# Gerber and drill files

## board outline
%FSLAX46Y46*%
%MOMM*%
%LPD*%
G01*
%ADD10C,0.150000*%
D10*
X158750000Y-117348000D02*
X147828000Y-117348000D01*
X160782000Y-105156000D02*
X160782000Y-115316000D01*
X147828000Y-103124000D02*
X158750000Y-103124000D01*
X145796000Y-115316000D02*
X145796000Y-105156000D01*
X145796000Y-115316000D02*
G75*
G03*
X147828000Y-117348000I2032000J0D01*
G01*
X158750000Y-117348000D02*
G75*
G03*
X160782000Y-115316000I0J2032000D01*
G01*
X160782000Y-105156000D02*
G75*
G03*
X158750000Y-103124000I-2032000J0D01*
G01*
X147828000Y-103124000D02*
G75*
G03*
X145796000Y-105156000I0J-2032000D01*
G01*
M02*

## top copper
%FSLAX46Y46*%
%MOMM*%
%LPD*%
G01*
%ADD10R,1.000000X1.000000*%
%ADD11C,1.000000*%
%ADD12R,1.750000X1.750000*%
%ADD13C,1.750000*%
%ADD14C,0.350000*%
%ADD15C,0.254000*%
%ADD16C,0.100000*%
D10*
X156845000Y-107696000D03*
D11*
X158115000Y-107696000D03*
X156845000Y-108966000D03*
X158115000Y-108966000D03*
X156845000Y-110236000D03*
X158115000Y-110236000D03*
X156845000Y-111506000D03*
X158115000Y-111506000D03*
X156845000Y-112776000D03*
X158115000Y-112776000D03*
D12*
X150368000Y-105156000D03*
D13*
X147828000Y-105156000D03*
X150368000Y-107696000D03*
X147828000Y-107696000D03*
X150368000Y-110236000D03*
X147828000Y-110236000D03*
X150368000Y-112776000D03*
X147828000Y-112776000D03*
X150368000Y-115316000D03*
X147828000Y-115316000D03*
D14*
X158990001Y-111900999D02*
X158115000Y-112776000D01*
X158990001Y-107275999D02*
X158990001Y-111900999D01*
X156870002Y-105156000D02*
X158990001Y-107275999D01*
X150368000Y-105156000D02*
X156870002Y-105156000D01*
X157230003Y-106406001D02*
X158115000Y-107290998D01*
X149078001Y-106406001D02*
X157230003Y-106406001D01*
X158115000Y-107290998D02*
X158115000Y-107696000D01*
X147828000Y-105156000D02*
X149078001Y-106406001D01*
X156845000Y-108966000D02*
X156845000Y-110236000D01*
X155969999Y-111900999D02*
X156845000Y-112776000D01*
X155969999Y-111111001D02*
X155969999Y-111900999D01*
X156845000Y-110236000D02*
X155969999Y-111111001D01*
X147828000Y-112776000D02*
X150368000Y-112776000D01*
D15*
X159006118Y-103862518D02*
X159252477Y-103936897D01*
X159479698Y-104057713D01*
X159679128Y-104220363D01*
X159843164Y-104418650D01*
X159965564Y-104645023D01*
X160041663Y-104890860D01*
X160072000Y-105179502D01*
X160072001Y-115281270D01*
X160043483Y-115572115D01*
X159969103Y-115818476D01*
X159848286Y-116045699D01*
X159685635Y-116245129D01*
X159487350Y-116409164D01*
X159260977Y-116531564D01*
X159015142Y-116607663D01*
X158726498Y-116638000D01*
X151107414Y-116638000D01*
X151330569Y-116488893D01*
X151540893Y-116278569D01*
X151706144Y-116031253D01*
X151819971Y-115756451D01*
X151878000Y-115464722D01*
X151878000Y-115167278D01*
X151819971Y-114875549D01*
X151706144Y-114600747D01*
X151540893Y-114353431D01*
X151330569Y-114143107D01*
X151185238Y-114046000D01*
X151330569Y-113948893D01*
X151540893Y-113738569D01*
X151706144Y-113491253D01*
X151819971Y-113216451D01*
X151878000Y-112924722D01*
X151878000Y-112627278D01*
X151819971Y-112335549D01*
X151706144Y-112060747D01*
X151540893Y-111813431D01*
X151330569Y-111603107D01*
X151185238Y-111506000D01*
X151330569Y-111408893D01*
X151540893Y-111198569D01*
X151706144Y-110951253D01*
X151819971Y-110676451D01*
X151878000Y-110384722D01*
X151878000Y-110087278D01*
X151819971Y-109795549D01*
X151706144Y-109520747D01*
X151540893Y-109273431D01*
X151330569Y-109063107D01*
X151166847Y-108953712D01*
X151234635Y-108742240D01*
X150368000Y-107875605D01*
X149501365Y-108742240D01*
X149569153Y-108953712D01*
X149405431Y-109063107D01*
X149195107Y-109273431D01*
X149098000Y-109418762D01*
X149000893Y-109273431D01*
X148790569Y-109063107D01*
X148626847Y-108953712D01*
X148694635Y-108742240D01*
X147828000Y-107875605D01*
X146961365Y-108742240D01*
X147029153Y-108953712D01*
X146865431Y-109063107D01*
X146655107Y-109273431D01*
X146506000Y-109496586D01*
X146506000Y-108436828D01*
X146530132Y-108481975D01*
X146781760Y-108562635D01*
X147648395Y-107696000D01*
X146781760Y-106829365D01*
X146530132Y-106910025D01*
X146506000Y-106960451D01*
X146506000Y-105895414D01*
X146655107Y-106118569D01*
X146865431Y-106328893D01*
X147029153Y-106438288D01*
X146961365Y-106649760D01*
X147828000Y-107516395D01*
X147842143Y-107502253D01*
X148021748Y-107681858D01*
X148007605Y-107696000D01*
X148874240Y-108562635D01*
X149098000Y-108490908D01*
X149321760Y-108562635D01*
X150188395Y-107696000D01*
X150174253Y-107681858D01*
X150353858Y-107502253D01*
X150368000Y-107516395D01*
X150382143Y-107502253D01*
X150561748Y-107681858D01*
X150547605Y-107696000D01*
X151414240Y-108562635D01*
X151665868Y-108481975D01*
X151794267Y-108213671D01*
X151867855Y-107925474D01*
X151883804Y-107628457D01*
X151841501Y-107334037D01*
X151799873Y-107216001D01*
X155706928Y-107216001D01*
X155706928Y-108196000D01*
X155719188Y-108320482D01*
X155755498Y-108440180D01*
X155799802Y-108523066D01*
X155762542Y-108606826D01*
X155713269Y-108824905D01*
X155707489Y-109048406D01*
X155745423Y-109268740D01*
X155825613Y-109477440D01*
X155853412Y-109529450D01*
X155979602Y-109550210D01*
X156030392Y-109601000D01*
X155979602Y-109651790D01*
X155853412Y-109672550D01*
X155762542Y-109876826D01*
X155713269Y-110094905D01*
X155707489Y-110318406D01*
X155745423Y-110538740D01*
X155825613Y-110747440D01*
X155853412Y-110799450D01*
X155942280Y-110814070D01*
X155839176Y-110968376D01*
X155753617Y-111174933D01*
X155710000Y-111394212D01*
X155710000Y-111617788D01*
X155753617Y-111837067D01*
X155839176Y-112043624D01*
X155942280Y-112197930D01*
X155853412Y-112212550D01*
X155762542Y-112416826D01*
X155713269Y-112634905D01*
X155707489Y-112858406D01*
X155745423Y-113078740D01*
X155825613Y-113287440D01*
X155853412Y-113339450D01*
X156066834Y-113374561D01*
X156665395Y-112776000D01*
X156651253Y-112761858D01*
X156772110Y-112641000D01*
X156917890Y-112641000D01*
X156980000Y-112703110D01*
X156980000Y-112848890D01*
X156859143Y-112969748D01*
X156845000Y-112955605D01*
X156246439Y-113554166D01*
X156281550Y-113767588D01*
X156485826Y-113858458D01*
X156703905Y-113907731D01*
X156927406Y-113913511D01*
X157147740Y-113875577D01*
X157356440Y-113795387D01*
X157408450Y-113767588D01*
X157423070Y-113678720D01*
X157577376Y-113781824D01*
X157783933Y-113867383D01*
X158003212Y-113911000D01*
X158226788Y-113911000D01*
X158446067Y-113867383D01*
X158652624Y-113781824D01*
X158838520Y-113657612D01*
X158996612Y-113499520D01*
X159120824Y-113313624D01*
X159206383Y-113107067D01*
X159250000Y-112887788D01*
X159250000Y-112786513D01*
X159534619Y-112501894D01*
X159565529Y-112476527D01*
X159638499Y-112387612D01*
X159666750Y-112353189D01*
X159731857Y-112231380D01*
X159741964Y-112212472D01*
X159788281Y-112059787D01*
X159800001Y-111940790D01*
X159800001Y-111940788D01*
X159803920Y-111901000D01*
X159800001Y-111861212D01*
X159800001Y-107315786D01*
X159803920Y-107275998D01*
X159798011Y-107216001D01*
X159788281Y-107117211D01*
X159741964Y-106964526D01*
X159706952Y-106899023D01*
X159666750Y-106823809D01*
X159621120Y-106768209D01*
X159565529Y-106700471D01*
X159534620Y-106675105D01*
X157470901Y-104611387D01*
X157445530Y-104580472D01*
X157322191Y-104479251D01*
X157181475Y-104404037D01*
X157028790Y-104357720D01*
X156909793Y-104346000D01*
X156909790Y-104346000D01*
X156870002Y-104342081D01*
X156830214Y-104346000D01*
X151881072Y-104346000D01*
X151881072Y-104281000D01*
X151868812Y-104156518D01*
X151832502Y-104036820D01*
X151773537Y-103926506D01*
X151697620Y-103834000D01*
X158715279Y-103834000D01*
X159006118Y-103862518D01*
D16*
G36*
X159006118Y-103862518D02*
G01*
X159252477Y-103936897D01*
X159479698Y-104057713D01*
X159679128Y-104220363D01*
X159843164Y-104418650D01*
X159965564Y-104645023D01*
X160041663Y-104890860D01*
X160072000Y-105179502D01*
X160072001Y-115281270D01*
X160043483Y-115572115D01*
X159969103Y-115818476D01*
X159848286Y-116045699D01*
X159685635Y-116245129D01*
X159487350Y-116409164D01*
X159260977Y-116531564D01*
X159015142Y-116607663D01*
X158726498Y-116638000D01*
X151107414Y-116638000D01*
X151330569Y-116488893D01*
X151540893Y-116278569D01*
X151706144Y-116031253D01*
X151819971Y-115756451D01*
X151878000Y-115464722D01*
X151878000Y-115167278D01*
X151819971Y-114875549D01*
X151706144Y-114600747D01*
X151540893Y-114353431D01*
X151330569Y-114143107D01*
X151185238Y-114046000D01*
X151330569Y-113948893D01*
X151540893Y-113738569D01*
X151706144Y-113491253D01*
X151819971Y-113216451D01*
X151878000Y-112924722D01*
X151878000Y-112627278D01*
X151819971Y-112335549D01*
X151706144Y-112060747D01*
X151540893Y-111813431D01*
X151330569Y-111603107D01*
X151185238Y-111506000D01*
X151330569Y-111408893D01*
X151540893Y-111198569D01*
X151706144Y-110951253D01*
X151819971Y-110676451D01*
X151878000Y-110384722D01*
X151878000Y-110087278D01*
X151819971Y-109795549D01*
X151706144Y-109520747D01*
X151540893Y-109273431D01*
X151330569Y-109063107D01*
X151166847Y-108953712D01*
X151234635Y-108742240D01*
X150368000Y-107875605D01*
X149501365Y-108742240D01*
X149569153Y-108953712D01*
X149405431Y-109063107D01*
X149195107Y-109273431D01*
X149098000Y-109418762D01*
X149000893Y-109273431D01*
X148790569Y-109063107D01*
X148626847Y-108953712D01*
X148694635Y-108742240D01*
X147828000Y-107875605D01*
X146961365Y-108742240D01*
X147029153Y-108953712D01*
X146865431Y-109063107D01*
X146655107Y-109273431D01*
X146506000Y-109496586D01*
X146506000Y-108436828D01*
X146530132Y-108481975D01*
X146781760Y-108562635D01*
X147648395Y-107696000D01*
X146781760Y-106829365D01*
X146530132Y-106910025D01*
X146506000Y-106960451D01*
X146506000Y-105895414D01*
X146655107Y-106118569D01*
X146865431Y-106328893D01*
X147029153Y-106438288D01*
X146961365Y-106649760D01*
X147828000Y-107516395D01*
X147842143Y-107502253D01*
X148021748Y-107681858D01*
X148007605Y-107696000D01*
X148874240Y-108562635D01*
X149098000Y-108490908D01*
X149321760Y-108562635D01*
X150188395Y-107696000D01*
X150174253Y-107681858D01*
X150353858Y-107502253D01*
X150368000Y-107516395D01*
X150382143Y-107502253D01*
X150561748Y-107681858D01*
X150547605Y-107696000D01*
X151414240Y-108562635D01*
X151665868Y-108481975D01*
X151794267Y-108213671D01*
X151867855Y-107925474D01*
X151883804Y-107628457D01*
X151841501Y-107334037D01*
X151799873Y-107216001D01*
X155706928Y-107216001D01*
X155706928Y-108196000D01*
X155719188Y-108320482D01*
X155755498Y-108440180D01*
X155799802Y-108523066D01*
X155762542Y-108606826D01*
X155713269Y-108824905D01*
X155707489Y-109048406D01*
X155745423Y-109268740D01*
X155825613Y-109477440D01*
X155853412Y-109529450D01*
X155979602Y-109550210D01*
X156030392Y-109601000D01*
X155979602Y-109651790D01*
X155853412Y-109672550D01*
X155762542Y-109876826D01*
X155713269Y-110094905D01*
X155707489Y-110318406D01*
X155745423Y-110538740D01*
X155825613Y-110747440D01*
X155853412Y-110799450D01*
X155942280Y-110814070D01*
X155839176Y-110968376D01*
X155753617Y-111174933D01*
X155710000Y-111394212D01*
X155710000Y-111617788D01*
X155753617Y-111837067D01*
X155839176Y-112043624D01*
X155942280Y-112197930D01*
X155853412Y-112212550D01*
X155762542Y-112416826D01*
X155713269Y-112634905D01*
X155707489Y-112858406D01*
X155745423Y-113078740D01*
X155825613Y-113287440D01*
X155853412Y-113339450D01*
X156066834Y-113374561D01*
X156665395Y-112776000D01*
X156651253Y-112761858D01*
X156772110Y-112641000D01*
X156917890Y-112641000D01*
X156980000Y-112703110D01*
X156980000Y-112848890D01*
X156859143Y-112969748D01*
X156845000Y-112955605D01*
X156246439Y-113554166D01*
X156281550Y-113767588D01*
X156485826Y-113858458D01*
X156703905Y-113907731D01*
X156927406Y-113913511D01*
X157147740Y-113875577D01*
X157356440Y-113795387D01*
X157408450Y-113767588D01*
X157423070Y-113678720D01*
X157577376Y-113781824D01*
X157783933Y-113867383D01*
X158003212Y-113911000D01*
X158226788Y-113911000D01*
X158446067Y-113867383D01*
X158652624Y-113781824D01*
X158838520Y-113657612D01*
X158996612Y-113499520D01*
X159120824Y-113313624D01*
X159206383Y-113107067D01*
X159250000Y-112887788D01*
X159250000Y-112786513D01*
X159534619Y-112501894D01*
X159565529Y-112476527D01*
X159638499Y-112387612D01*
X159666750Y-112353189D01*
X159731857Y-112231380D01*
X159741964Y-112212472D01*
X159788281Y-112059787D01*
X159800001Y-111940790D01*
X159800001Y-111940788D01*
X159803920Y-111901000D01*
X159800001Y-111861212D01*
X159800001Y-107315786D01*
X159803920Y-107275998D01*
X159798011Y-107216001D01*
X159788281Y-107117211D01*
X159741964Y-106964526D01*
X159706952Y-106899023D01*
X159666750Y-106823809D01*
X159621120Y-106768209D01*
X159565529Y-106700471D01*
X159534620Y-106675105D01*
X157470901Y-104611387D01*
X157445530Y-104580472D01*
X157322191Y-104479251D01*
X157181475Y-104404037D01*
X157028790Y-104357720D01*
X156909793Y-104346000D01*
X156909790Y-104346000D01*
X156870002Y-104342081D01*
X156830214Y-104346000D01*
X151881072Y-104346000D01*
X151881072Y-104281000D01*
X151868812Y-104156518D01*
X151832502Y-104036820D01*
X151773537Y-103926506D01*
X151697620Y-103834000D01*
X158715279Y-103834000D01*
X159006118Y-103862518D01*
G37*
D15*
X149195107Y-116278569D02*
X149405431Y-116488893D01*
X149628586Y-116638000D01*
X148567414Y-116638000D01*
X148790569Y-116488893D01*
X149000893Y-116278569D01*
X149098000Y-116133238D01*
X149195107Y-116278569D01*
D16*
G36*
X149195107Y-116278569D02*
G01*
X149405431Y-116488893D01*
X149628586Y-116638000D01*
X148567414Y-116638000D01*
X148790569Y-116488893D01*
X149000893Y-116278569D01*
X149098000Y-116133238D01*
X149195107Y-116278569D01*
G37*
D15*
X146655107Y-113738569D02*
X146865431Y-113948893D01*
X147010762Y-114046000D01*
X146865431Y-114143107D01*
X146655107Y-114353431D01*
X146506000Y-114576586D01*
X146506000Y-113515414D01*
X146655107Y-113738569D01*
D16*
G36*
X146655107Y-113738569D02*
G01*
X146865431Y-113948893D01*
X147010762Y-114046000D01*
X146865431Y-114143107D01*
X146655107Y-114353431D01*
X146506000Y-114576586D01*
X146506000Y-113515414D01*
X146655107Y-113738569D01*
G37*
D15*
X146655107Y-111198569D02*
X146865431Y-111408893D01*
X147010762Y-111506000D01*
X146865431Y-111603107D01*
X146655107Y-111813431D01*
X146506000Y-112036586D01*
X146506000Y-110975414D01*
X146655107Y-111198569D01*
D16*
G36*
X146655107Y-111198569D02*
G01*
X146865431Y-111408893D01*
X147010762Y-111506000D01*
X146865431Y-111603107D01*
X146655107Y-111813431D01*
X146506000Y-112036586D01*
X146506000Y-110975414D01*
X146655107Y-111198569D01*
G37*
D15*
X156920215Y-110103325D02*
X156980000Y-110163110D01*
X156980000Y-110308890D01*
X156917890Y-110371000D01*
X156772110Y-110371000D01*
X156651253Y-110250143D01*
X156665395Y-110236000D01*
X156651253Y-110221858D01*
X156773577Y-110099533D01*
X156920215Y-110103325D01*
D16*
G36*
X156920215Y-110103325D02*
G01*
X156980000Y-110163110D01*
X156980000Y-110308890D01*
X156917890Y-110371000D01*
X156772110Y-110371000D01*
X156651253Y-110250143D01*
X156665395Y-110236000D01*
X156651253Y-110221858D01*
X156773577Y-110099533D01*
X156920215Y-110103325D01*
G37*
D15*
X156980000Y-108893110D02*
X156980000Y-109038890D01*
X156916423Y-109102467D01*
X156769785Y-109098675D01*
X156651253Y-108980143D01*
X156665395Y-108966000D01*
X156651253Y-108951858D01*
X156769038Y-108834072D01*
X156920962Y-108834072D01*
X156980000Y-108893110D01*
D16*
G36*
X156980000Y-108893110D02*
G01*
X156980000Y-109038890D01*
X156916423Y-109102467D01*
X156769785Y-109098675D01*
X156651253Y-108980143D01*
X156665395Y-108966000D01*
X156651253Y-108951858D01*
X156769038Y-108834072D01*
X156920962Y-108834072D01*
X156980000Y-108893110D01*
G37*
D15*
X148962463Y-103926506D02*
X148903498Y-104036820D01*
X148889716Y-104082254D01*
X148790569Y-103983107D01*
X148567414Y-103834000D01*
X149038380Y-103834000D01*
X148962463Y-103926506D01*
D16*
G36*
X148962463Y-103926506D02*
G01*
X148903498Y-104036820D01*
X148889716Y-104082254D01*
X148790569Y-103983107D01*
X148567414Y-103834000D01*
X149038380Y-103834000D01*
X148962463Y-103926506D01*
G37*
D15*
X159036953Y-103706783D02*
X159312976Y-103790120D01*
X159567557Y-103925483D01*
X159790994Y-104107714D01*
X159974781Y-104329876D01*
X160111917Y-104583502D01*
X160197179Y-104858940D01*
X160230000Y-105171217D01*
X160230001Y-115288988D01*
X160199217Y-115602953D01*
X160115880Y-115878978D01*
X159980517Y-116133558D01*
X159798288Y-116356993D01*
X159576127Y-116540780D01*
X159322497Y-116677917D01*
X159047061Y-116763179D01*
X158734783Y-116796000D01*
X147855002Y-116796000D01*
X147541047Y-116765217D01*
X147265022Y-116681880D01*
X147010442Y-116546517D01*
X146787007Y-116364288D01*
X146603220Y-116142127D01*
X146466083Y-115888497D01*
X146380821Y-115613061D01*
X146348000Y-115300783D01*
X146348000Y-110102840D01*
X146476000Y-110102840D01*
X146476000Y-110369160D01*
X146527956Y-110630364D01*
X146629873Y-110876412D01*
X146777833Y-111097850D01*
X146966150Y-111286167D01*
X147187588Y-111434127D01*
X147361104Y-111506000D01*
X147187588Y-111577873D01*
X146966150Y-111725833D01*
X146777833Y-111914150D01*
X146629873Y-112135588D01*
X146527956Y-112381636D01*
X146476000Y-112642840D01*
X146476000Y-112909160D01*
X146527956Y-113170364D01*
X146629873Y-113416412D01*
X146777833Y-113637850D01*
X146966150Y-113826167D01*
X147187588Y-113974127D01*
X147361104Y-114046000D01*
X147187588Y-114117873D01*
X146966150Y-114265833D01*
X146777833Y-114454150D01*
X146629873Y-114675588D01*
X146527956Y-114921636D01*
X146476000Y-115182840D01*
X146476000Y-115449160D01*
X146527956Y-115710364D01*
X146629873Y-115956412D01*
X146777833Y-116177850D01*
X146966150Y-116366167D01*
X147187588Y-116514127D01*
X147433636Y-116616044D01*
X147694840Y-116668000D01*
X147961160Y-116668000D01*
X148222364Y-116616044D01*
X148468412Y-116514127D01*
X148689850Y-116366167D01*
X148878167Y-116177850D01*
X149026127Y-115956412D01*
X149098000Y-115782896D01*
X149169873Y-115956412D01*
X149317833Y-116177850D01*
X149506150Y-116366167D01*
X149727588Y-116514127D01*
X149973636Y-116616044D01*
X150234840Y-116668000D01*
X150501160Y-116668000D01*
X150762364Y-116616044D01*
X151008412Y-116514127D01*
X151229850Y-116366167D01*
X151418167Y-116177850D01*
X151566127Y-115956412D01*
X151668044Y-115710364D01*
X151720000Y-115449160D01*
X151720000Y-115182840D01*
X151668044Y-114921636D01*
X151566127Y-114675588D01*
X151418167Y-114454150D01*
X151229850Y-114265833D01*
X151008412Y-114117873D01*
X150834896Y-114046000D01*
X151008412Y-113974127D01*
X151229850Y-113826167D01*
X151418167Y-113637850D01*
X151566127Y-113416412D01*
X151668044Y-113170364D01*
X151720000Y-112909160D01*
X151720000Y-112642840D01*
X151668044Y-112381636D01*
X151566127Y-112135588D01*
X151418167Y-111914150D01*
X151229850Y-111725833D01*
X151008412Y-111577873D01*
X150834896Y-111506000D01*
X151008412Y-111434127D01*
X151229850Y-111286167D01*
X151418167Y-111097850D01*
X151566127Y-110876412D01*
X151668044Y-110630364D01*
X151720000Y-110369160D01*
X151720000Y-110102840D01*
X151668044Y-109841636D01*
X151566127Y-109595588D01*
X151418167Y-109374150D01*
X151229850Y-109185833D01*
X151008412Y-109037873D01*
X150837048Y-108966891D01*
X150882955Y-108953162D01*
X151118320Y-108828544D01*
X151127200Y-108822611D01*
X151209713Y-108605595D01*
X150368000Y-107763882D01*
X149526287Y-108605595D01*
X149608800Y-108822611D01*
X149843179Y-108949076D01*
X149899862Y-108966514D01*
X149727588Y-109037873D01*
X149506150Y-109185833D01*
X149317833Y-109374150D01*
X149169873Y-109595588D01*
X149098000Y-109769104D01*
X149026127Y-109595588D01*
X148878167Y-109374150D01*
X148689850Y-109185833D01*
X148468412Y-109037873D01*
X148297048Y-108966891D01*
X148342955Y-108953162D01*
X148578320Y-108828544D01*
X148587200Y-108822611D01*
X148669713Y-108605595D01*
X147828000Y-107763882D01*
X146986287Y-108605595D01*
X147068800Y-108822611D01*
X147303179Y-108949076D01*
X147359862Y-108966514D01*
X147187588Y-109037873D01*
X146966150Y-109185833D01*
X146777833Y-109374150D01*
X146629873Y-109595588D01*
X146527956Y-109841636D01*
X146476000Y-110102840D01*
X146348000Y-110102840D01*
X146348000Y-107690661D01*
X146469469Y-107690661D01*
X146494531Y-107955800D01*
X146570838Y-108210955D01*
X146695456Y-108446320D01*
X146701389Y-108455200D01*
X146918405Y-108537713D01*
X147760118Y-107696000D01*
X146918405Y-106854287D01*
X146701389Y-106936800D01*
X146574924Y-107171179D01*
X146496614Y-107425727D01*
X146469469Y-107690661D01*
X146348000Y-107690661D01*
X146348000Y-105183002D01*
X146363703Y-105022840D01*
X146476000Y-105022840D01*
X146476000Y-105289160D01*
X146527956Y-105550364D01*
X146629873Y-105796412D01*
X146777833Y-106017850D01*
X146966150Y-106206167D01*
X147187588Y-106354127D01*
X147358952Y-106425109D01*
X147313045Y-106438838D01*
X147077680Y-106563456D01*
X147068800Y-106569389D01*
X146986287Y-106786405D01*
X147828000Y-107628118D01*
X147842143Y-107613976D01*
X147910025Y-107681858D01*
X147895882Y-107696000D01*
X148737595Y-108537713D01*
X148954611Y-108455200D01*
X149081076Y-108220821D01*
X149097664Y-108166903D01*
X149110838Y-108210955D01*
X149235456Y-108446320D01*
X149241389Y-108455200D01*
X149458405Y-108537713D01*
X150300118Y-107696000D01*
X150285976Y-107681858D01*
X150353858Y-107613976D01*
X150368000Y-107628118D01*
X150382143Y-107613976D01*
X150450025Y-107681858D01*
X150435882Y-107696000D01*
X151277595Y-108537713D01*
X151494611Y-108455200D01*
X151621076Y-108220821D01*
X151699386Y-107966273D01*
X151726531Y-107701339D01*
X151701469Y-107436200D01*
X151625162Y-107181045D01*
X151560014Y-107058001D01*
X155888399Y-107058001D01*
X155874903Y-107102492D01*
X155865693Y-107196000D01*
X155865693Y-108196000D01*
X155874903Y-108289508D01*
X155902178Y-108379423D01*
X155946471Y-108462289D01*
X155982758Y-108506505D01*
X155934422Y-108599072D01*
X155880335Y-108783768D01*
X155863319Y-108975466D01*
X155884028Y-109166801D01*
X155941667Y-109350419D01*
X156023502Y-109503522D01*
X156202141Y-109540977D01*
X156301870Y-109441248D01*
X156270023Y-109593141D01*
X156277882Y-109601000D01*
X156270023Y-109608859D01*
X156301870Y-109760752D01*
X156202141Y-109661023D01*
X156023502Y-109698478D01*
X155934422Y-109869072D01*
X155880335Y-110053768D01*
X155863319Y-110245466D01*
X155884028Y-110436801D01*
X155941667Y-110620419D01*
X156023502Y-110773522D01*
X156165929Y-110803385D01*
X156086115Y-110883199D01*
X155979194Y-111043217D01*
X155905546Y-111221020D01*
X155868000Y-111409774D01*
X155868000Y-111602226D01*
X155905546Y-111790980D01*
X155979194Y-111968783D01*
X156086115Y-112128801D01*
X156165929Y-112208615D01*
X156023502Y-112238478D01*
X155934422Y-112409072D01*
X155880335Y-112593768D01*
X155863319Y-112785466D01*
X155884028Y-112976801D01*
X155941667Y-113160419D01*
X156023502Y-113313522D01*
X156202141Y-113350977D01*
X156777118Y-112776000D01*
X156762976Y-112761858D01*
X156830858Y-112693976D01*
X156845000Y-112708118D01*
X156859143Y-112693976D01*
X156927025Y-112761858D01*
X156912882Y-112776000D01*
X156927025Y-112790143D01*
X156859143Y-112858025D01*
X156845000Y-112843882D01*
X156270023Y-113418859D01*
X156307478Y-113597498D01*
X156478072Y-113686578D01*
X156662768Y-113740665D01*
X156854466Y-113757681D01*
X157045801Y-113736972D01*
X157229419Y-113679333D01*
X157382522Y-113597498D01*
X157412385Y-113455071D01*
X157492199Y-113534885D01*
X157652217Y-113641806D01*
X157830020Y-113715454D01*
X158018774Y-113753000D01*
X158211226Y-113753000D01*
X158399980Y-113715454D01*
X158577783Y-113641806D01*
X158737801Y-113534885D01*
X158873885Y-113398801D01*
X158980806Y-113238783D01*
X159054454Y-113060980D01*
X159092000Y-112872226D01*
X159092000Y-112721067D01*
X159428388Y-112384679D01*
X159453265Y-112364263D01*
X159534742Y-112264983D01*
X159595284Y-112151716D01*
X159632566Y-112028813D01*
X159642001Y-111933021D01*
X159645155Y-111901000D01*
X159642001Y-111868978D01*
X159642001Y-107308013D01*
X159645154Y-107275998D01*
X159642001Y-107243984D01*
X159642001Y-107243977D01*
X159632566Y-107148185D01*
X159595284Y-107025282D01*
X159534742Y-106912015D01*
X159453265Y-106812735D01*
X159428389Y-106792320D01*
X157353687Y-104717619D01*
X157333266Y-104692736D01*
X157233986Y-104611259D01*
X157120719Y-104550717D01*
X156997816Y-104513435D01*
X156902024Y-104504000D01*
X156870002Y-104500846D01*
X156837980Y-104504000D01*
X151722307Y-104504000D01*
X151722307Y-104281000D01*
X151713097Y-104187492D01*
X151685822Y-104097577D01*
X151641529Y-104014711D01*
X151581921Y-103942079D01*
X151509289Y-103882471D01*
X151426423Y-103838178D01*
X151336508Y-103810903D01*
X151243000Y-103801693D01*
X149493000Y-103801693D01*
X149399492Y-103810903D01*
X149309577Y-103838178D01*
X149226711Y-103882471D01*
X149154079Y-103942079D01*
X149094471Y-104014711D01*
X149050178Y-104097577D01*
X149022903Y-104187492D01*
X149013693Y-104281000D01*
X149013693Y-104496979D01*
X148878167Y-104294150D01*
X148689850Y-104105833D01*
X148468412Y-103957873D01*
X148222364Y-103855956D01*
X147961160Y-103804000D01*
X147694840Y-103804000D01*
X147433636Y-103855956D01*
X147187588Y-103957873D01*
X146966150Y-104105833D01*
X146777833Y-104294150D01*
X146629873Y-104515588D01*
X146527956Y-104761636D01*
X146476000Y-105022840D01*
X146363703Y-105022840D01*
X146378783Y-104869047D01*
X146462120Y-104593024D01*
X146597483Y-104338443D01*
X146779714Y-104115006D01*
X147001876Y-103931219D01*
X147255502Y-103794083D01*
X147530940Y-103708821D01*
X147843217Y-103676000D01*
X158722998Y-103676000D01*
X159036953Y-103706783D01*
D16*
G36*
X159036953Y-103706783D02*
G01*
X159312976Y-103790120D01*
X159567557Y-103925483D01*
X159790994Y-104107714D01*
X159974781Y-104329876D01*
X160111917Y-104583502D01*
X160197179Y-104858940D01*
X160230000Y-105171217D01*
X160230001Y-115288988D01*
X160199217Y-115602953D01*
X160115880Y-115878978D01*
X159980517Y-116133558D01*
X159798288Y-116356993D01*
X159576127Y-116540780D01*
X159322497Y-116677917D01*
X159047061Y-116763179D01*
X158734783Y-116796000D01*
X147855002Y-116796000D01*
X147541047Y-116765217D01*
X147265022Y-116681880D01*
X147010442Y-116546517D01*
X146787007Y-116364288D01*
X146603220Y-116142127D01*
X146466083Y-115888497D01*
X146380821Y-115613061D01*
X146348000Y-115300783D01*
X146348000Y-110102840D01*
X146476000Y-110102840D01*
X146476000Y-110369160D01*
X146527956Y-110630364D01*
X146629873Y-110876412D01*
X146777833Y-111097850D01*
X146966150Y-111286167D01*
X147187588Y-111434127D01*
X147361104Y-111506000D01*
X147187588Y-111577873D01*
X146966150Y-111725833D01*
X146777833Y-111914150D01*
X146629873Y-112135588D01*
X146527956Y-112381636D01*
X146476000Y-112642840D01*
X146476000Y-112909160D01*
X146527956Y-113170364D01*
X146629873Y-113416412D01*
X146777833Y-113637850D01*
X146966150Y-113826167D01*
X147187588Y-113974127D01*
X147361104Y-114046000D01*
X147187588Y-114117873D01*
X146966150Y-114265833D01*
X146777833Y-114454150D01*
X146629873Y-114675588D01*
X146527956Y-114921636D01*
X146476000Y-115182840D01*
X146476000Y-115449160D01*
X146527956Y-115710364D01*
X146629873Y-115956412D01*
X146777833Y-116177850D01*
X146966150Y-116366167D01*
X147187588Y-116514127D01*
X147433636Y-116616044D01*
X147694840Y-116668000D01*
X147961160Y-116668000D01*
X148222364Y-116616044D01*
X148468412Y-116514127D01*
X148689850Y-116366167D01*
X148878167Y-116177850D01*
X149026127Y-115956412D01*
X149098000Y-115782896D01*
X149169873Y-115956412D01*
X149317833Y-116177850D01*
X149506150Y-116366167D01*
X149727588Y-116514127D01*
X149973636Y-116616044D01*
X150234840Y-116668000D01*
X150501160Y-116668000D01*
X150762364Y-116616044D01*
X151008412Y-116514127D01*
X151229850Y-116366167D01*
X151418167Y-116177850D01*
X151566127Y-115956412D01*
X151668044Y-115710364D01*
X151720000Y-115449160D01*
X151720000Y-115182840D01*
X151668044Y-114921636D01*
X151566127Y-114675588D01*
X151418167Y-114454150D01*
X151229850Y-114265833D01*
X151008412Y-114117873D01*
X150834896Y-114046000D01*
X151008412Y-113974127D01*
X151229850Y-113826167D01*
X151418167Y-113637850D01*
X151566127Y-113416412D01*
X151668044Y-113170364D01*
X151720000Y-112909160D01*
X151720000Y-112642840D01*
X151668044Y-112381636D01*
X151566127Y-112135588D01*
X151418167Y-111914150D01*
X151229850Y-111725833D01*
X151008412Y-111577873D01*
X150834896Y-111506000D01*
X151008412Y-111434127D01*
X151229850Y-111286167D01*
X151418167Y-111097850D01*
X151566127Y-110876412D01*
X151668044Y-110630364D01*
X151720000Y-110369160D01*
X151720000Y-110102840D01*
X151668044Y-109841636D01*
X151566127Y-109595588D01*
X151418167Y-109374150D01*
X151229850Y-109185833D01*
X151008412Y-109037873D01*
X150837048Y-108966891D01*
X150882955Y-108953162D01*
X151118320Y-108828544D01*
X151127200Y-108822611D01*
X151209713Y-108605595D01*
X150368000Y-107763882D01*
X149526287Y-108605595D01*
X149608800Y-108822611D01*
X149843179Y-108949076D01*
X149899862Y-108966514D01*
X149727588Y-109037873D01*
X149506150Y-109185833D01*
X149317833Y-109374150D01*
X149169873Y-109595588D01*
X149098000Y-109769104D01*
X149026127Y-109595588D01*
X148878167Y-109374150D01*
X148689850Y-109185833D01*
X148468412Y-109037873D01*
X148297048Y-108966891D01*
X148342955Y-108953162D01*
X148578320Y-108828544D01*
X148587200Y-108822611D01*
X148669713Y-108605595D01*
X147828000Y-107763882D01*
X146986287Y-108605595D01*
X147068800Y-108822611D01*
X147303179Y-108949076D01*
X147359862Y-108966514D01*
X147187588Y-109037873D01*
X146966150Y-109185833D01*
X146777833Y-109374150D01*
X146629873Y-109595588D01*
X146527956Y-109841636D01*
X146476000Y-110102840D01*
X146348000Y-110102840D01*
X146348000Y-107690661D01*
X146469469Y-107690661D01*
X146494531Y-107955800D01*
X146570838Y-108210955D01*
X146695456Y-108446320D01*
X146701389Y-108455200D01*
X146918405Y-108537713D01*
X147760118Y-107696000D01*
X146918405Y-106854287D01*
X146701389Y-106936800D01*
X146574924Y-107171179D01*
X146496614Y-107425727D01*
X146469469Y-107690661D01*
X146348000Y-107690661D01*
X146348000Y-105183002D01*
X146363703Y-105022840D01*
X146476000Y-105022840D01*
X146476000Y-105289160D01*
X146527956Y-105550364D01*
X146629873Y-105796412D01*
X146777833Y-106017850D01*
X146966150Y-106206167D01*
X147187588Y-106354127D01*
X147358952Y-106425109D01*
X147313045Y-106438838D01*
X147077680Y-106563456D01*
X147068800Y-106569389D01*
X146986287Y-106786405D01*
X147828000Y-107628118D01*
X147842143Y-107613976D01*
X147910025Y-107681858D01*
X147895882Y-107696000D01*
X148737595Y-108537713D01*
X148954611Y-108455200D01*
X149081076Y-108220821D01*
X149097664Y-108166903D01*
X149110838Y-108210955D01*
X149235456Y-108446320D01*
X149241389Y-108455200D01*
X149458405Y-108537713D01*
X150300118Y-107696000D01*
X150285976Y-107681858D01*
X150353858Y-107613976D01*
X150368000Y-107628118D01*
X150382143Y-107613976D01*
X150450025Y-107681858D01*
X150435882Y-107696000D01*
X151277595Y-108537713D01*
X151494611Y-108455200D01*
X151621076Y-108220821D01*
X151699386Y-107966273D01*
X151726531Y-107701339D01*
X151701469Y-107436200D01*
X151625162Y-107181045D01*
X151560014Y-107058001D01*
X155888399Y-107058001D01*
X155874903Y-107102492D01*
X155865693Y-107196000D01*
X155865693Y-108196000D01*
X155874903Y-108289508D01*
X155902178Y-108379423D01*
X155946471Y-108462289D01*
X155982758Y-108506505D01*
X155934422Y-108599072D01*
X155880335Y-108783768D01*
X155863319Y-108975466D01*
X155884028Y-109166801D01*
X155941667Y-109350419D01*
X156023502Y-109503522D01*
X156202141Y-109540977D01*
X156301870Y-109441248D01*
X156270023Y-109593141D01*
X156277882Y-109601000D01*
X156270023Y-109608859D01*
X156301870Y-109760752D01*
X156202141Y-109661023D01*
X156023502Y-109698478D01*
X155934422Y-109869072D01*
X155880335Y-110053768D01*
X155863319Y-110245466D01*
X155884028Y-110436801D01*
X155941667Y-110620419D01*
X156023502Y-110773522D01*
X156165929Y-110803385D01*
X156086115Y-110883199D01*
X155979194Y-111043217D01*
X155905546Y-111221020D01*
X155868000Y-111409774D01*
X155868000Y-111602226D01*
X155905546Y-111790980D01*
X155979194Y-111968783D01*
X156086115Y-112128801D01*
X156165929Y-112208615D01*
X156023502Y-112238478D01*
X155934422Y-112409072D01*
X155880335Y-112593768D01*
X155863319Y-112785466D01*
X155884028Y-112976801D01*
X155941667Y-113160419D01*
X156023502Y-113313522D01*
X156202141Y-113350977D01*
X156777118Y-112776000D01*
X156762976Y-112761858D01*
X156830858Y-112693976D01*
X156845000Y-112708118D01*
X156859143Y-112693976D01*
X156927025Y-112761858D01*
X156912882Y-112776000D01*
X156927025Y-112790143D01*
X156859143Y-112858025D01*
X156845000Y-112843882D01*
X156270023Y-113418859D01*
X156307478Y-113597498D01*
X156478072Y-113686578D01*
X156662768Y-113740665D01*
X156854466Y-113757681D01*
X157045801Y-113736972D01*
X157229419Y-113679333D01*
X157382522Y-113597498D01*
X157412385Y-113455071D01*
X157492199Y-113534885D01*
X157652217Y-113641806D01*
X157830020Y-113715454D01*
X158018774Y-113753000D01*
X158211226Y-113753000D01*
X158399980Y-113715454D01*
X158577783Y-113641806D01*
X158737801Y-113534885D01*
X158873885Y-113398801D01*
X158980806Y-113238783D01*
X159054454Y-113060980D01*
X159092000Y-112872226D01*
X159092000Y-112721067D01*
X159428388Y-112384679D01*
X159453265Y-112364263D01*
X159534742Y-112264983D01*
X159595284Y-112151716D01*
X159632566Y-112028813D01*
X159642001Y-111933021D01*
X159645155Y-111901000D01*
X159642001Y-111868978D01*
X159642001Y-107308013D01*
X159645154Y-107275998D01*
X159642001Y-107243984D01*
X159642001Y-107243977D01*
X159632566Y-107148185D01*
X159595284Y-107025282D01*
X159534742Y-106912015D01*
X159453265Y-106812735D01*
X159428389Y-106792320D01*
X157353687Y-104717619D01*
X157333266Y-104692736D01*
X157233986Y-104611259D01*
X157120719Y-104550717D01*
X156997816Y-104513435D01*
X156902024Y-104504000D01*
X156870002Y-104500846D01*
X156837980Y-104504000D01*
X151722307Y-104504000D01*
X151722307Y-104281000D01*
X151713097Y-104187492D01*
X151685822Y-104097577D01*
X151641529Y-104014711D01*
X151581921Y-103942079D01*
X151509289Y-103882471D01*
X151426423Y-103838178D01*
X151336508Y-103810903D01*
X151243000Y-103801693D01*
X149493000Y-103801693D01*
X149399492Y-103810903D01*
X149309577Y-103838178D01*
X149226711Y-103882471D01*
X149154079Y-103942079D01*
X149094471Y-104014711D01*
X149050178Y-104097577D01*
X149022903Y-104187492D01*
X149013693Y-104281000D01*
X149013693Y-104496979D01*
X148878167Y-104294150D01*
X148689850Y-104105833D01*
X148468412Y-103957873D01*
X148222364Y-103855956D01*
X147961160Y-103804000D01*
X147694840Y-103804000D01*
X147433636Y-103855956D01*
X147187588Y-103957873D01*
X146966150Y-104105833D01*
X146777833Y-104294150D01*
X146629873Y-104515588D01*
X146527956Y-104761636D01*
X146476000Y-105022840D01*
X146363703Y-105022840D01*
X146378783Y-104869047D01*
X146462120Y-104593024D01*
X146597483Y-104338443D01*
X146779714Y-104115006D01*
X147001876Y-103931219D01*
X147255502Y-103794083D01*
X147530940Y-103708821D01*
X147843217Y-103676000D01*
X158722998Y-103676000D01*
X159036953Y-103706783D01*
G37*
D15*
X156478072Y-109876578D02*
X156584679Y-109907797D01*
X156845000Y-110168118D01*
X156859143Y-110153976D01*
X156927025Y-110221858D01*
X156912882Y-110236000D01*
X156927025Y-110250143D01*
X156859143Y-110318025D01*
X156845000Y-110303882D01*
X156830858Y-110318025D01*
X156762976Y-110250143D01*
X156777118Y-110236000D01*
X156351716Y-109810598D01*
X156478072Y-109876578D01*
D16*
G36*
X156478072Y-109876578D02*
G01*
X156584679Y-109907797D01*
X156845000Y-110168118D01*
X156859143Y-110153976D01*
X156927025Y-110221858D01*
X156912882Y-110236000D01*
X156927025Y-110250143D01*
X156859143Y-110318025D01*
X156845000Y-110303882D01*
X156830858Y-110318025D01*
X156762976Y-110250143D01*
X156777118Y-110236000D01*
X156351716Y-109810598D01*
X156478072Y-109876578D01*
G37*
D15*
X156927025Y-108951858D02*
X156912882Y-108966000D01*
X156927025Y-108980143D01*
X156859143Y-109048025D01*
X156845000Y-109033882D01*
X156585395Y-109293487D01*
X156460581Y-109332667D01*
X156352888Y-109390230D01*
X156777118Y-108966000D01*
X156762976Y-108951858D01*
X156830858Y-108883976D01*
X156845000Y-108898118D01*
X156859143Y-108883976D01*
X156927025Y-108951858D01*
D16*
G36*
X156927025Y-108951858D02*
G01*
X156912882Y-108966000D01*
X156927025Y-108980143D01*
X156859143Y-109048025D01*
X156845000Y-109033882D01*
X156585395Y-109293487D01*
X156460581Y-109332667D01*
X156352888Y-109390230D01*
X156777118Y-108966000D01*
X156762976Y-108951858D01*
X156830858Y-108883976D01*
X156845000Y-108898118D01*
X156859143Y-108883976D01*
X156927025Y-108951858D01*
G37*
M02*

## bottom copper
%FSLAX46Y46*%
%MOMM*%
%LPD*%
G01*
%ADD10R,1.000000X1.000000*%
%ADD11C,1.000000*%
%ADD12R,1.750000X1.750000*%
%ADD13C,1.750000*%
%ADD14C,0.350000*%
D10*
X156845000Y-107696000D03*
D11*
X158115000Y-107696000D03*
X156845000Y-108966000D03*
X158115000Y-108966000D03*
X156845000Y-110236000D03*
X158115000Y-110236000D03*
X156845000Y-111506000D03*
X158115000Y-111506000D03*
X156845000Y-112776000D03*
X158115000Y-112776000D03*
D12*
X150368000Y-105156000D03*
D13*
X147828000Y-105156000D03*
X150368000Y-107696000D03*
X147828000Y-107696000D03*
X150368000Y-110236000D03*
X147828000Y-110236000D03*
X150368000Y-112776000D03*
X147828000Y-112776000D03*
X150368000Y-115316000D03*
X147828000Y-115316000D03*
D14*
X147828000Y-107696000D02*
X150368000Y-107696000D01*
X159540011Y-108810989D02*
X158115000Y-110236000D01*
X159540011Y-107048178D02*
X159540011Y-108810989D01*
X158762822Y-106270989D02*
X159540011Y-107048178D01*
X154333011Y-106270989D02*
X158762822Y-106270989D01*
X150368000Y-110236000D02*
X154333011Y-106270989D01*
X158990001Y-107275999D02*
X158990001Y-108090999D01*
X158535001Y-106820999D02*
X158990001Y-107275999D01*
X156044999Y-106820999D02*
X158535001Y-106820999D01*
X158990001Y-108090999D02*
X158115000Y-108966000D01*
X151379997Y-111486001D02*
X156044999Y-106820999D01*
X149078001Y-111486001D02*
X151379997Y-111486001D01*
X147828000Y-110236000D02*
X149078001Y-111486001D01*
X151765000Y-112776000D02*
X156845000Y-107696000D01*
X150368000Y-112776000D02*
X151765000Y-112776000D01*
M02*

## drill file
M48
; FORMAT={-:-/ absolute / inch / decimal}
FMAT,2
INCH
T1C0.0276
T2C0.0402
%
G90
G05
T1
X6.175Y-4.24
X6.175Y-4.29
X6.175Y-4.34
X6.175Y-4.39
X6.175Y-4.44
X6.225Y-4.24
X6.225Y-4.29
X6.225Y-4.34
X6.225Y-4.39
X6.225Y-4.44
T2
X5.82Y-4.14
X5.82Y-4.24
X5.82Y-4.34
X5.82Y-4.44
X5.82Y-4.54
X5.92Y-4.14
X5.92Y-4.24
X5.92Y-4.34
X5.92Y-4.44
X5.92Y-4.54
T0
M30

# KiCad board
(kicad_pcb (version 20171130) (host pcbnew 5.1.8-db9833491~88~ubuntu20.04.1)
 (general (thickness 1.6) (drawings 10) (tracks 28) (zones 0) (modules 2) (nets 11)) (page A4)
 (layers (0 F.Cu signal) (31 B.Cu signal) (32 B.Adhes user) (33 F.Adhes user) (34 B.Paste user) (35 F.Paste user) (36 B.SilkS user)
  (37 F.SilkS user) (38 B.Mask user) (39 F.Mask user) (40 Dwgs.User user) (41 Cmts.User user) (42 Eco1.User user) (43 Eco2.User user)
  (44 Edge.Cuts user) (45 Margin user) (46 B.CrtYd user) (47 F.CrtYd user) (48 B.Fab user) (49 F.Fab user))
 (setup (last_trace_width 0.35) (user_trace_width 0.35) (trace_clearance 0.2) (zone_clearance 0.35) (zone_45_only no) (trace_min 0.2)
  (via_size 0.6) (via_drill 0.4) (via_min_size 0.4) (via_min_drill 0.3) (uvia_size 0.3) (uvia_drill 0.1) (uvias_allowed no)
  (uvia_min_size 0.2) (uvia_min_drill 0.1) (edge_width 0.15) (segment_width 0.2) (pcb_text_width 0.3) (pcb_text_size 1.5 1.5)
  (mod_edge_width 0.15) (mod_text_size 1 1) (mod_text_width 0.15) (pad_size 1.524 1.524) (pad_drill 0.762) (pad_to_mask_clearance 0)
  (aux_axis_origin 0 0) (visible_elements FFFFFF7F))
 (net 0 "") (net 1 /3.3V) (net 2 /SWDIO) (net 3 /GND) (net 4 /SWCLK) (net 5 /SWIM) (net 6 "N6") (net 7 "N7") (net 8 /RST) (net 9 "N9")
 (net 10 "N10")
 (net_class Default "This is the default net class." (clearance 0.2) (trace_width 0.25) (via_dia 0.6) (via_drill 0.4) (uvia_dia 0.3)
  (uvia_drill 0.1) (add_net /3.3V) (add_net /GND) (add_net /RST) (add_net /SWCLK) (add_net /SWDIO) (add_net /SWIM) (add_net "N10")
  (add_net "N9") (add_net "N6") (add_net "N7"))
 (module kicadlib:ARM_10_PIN (layer F.Cu) (at 157.48 110.236)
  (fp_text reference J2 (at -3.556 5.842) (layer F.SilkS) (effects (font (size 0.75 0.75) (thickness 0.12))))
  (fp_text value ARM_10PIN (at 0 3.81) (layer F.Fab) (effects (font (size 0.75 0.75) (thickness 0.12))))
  (pad 1 thru_hole rect (at -0.635 -2.54) (size 1 1) (drill 0.70104) (layers *.Cu *.Mask F.SilkS) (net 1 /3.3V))
  (pad 2 thru_hole circle (at 0.635 -2.54) (size 1 1) (drill 0.70104) (layers *.Cu *.Mask F.SilkS) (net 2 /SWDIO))
  (pad 3 thru_hole circle (at -0.635 -1.27) (size 1 1) (drill 0.70104) (layers *.Cu *.Mask F.SilkS) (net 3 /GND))
  (pad 4 thru_hole circle (at 0.635 -1.27) (size 1 1) (drill 0.70104) (layers *.Cu *.Mask F.SilkS) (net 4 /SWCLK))
  (pad 5 thru_hole circle (at -0.635 0) (size 1 1) (drill 0.70104) (layers *.Cu *.Mask F.SilkS) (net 3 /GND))
  (pad 6 thru_hole circle (at 0.635 0) (size 1 1) (drill 0.70104) (layers *.Cu *.Mask F.SilkS) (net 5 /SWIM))
  (pad 7 thru_hole circle (at -0.635 1.27) (size 1 1) (drill 0.70104) (layers *.Cu *.Mask F.SilkS) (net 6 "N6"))
  (pad 8 thru_hole circle (at 0.635 1.27) (size 1 1) (drill 0.70104) (layers *.Cu *.Mask F.SilkS) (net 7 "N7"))
  (pad 9 thru_hole circle (at -0.635 2.54) (size 1 1) (drill 0.70104) (layers *.Cu *.Mask F.SilkS) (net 3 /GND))
  (pad 10 thru_hole circle (at 0.635 2.54) (size 1 1) (drill 0.70104) (layers *.Cu *.Mask F.SilkS) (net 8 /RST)))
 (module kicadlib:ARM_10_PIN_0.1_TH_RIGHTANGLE (layer F.Cu) (at 150.368 105.156)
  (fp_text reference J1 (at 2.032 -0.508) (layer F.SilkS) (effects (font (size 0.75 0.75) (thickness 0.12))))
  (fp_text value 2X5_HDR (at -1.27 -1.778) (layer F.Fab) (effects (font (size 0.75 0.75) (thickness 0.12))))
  (pad 1 thru_hole rect (at 0 0) (size 1.75 1.75) (drill 1.02) (layers *.Cu *.Mask F.SilkS) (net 8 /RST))
  (pad 2 thru_hole circle (at -2.54 0) (size 1.75 1.75) (drill 1.02) (layers *.Cu *.Mask F.SilkS) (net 2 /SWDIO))
  (pad 3 thru_hole circle (at 0 2.54) (size 1.75 1.75) (drill 1.02) (layers *.Cu *.Mask F.SilkS) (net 3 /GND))
  (pad 4 thru_hole circle (at -2.54 2.54) (size 1.75 1.75) (drill 1.02) (layers *.Cu *.Mask F.SilkS) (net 3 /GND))
  (pad 5 thru_hole circle (at 0 5.08) (size 1.75 1.75) (drill 1.02) (layers *.Cu *.Mask F.SilkS) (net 5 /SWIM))
  (pad 6 thru_hole circle (at -2.54 5.08) (size 1.75 1.75) (drill 1.02) (layers *.Cu *.Mask F.SilkS) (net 4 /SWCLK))
  (pad 7 thru_hole circle (at 0 7.62) (size 1.75 1.75) (drill 1.02) (layers *.Cu *.Mask F.SilkS) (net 1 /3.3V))
  (pad 8 thru_hole circle (at -2.54 7.62) (size 1.75 1.75) (drill 1.02) (layers *.Cu *.Mask F.SilkS) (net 1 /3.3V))
  (pad 9 thru_hole circle (at 0 10.16) (size 1.75 1.75) (drill 1.02) (layers *.Cu *.Mask F.SilkS) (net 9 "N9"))
  (pad 10 thru_hole circle (at -2.54 10.16) (size 1.75 1.75) (drill 1.02) (layers *.Cu *.Mask F.SilkS) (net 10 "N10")))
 (gr_line (start 158.75 117.348) (end 147.828 117.348) (angle 90) (layer Edge.Cuts) (width 0.15))
 (gr_line (start 160.782 105.156) (end 160.782 115.316) (angle 90) (layer Edge.Cuts) (width 0.15))
 (gr_line (start 147.828 103.124) (end 158.75 103.124) (angle 90) (layer Edge.Cuts) (width 0.15))
 (gr_line (start 145.796 115.316) (end 145.796 105.156) (angle 90) (layer Edge.Cuts) (width 0.15))
 (gr_arc (start 147.828 115.316) (end 147.828 117.348) (angle 90) (layer Edge.Cuts) (width 0.15))
 (gr_arc (start 158.75 115.316) (end 160.782 115.316) (angle 90) (layer Edge.Cuts) (width 0.15))
 (gr_arc (start 158.75 105.156) (end 158.75 103.124) (angle 90) (layer Edge.Cuts) (width 0.15))
 (gr_arc (start 147.828 105.156) (end 145.796 105.156) (angle 90) (layer Edge.Cuts) (width 0.15))
 (segment (start 158.990001 111.900999) (end 158.115 112.776) (width 0.35) (layer F.Cu) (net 8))
 (segment (start 158.990001 107.275999) (end 158.990001 111.900999) (width 0.35) (layer F.Cu) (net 8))
 (segment (start 156.870002 105.156) (end 158.990001 107.275999) (width 0.35) (layer F.Cu) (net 8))
 (segment (start 150.368 105.156) (end 156.870002 105.156) (width 0.35) (layer F.Cu) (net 8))
 (segment (start 157.230003 106.406001) (end 158.115 107.290998) (width 0.35) (layer F.Cu) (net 2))
 (segment (start 149.078001 106.406001) (end 157.230003 106.406001) (width 0.35) (layer F.Cu) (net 2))
 (segment (start 158.115 107.290998) (end 158.115 107.696) (width 0.35) (layer F.Cu) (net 2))
 (segment (start 147.828 105.156) (end 149.078001 106.406001) (width 0.35) (layer F.Cu) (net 2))
 (segment (start 147.828 107.696) (end 150.368 107.696) (width 0.35) (layer B.Cu) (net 3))
 (segment (start 156.845 108.966) (end 156.845 110.236) (width 0.35) (layer F.Cu) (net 3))
 (segment (start 155.969999 111.900999) (end 156.845 112.776) (width 0.35) (layer F.Cu) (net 3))
 (segment (start 155.969999 111.111001) (end 155.969999 111.900999) (width 0.35) (layer F.Cu) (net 3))
 (segment (start 156.845 110.236) (end 155.969999 111.111001) (width 0.35) (layer F.Cu) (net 3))
 (segment (start 159.540011 108.810989) (end 158.115 110.236) (width 0.35) (layer B.Cu) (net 5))
 (segment (start 159.540011 107.048178) (end 159.540011 108.810989) (width 0.35) (layer B.Cu) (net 5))
 (segment (start 158.762822 106.270989) (end 159.540011 107.048178) (width 0.35) (layer B.Cu) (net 5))
 (segment (start 154.333011 106.270989) (end 158.762822 106.270989) (width 0.35) (layer B.Cu) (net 5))
 (segment (start 150.368 110.236) (end 154.333011 106.270989) (width 0.35) (layer B.Cu) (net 5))
 (segment (start 158.990001 107.275999) (end 158.990001 108.090999) (width 0.35) (layer B.Cu) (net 4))
 (segment (start 158.535001 106.820999) (end 158.990001 107.275999) (width 0.35) (layer B.Cu) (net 4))
 (segment (start 156.044999 106.820999) (end 158.535001 106.820999) (width 0.35) (layer B.Cu) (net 4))
 (segment (start 158.990001 108.090999) (end 158.115 108.966) (width 0.35) (layer B.Cu) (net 4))
 (segment (start 151.379997 111.486001) (end 156.044999 106.820999) (width 0.35) (layer B.Cu) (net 4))
 (segment (start 149.078001 111.486001) (end 151.379997 111.486001) (width 0.35) (layer B.Cu) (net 4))
 (segment (start 147.828 110.236) (end 149.078001 111.486001) (width 0.35) (layer B.Cu) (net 4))
 (segment (start 147.828 112.776) (end 150.368 112.776) (width 0.35) (layer F.Cu) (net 1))
 (segment (start 151.765 112.776) (end 156.845 107.696) (width 0.35) (layer B.Cu) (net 1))
 (segment (start 150.368 112.776) (end 151.765 112.776) (width 0.35) (layer B.Cu) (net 1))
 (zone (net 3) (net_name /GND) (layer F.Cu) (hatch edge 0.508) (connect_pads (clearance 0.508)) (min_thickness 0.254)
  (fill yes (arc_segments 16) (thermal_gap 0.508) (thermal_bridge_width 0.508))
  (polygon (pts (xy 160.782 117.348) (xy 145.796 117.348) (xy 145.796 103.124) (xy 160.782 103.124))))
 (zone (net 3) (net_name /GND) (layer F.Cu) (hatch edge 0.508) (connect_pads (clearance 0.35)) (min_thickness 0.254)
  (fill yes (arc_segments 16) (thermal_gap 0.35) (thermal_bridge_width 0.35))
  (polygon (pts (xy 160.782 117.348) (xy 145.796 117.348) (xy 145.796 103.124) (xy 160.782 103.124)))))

